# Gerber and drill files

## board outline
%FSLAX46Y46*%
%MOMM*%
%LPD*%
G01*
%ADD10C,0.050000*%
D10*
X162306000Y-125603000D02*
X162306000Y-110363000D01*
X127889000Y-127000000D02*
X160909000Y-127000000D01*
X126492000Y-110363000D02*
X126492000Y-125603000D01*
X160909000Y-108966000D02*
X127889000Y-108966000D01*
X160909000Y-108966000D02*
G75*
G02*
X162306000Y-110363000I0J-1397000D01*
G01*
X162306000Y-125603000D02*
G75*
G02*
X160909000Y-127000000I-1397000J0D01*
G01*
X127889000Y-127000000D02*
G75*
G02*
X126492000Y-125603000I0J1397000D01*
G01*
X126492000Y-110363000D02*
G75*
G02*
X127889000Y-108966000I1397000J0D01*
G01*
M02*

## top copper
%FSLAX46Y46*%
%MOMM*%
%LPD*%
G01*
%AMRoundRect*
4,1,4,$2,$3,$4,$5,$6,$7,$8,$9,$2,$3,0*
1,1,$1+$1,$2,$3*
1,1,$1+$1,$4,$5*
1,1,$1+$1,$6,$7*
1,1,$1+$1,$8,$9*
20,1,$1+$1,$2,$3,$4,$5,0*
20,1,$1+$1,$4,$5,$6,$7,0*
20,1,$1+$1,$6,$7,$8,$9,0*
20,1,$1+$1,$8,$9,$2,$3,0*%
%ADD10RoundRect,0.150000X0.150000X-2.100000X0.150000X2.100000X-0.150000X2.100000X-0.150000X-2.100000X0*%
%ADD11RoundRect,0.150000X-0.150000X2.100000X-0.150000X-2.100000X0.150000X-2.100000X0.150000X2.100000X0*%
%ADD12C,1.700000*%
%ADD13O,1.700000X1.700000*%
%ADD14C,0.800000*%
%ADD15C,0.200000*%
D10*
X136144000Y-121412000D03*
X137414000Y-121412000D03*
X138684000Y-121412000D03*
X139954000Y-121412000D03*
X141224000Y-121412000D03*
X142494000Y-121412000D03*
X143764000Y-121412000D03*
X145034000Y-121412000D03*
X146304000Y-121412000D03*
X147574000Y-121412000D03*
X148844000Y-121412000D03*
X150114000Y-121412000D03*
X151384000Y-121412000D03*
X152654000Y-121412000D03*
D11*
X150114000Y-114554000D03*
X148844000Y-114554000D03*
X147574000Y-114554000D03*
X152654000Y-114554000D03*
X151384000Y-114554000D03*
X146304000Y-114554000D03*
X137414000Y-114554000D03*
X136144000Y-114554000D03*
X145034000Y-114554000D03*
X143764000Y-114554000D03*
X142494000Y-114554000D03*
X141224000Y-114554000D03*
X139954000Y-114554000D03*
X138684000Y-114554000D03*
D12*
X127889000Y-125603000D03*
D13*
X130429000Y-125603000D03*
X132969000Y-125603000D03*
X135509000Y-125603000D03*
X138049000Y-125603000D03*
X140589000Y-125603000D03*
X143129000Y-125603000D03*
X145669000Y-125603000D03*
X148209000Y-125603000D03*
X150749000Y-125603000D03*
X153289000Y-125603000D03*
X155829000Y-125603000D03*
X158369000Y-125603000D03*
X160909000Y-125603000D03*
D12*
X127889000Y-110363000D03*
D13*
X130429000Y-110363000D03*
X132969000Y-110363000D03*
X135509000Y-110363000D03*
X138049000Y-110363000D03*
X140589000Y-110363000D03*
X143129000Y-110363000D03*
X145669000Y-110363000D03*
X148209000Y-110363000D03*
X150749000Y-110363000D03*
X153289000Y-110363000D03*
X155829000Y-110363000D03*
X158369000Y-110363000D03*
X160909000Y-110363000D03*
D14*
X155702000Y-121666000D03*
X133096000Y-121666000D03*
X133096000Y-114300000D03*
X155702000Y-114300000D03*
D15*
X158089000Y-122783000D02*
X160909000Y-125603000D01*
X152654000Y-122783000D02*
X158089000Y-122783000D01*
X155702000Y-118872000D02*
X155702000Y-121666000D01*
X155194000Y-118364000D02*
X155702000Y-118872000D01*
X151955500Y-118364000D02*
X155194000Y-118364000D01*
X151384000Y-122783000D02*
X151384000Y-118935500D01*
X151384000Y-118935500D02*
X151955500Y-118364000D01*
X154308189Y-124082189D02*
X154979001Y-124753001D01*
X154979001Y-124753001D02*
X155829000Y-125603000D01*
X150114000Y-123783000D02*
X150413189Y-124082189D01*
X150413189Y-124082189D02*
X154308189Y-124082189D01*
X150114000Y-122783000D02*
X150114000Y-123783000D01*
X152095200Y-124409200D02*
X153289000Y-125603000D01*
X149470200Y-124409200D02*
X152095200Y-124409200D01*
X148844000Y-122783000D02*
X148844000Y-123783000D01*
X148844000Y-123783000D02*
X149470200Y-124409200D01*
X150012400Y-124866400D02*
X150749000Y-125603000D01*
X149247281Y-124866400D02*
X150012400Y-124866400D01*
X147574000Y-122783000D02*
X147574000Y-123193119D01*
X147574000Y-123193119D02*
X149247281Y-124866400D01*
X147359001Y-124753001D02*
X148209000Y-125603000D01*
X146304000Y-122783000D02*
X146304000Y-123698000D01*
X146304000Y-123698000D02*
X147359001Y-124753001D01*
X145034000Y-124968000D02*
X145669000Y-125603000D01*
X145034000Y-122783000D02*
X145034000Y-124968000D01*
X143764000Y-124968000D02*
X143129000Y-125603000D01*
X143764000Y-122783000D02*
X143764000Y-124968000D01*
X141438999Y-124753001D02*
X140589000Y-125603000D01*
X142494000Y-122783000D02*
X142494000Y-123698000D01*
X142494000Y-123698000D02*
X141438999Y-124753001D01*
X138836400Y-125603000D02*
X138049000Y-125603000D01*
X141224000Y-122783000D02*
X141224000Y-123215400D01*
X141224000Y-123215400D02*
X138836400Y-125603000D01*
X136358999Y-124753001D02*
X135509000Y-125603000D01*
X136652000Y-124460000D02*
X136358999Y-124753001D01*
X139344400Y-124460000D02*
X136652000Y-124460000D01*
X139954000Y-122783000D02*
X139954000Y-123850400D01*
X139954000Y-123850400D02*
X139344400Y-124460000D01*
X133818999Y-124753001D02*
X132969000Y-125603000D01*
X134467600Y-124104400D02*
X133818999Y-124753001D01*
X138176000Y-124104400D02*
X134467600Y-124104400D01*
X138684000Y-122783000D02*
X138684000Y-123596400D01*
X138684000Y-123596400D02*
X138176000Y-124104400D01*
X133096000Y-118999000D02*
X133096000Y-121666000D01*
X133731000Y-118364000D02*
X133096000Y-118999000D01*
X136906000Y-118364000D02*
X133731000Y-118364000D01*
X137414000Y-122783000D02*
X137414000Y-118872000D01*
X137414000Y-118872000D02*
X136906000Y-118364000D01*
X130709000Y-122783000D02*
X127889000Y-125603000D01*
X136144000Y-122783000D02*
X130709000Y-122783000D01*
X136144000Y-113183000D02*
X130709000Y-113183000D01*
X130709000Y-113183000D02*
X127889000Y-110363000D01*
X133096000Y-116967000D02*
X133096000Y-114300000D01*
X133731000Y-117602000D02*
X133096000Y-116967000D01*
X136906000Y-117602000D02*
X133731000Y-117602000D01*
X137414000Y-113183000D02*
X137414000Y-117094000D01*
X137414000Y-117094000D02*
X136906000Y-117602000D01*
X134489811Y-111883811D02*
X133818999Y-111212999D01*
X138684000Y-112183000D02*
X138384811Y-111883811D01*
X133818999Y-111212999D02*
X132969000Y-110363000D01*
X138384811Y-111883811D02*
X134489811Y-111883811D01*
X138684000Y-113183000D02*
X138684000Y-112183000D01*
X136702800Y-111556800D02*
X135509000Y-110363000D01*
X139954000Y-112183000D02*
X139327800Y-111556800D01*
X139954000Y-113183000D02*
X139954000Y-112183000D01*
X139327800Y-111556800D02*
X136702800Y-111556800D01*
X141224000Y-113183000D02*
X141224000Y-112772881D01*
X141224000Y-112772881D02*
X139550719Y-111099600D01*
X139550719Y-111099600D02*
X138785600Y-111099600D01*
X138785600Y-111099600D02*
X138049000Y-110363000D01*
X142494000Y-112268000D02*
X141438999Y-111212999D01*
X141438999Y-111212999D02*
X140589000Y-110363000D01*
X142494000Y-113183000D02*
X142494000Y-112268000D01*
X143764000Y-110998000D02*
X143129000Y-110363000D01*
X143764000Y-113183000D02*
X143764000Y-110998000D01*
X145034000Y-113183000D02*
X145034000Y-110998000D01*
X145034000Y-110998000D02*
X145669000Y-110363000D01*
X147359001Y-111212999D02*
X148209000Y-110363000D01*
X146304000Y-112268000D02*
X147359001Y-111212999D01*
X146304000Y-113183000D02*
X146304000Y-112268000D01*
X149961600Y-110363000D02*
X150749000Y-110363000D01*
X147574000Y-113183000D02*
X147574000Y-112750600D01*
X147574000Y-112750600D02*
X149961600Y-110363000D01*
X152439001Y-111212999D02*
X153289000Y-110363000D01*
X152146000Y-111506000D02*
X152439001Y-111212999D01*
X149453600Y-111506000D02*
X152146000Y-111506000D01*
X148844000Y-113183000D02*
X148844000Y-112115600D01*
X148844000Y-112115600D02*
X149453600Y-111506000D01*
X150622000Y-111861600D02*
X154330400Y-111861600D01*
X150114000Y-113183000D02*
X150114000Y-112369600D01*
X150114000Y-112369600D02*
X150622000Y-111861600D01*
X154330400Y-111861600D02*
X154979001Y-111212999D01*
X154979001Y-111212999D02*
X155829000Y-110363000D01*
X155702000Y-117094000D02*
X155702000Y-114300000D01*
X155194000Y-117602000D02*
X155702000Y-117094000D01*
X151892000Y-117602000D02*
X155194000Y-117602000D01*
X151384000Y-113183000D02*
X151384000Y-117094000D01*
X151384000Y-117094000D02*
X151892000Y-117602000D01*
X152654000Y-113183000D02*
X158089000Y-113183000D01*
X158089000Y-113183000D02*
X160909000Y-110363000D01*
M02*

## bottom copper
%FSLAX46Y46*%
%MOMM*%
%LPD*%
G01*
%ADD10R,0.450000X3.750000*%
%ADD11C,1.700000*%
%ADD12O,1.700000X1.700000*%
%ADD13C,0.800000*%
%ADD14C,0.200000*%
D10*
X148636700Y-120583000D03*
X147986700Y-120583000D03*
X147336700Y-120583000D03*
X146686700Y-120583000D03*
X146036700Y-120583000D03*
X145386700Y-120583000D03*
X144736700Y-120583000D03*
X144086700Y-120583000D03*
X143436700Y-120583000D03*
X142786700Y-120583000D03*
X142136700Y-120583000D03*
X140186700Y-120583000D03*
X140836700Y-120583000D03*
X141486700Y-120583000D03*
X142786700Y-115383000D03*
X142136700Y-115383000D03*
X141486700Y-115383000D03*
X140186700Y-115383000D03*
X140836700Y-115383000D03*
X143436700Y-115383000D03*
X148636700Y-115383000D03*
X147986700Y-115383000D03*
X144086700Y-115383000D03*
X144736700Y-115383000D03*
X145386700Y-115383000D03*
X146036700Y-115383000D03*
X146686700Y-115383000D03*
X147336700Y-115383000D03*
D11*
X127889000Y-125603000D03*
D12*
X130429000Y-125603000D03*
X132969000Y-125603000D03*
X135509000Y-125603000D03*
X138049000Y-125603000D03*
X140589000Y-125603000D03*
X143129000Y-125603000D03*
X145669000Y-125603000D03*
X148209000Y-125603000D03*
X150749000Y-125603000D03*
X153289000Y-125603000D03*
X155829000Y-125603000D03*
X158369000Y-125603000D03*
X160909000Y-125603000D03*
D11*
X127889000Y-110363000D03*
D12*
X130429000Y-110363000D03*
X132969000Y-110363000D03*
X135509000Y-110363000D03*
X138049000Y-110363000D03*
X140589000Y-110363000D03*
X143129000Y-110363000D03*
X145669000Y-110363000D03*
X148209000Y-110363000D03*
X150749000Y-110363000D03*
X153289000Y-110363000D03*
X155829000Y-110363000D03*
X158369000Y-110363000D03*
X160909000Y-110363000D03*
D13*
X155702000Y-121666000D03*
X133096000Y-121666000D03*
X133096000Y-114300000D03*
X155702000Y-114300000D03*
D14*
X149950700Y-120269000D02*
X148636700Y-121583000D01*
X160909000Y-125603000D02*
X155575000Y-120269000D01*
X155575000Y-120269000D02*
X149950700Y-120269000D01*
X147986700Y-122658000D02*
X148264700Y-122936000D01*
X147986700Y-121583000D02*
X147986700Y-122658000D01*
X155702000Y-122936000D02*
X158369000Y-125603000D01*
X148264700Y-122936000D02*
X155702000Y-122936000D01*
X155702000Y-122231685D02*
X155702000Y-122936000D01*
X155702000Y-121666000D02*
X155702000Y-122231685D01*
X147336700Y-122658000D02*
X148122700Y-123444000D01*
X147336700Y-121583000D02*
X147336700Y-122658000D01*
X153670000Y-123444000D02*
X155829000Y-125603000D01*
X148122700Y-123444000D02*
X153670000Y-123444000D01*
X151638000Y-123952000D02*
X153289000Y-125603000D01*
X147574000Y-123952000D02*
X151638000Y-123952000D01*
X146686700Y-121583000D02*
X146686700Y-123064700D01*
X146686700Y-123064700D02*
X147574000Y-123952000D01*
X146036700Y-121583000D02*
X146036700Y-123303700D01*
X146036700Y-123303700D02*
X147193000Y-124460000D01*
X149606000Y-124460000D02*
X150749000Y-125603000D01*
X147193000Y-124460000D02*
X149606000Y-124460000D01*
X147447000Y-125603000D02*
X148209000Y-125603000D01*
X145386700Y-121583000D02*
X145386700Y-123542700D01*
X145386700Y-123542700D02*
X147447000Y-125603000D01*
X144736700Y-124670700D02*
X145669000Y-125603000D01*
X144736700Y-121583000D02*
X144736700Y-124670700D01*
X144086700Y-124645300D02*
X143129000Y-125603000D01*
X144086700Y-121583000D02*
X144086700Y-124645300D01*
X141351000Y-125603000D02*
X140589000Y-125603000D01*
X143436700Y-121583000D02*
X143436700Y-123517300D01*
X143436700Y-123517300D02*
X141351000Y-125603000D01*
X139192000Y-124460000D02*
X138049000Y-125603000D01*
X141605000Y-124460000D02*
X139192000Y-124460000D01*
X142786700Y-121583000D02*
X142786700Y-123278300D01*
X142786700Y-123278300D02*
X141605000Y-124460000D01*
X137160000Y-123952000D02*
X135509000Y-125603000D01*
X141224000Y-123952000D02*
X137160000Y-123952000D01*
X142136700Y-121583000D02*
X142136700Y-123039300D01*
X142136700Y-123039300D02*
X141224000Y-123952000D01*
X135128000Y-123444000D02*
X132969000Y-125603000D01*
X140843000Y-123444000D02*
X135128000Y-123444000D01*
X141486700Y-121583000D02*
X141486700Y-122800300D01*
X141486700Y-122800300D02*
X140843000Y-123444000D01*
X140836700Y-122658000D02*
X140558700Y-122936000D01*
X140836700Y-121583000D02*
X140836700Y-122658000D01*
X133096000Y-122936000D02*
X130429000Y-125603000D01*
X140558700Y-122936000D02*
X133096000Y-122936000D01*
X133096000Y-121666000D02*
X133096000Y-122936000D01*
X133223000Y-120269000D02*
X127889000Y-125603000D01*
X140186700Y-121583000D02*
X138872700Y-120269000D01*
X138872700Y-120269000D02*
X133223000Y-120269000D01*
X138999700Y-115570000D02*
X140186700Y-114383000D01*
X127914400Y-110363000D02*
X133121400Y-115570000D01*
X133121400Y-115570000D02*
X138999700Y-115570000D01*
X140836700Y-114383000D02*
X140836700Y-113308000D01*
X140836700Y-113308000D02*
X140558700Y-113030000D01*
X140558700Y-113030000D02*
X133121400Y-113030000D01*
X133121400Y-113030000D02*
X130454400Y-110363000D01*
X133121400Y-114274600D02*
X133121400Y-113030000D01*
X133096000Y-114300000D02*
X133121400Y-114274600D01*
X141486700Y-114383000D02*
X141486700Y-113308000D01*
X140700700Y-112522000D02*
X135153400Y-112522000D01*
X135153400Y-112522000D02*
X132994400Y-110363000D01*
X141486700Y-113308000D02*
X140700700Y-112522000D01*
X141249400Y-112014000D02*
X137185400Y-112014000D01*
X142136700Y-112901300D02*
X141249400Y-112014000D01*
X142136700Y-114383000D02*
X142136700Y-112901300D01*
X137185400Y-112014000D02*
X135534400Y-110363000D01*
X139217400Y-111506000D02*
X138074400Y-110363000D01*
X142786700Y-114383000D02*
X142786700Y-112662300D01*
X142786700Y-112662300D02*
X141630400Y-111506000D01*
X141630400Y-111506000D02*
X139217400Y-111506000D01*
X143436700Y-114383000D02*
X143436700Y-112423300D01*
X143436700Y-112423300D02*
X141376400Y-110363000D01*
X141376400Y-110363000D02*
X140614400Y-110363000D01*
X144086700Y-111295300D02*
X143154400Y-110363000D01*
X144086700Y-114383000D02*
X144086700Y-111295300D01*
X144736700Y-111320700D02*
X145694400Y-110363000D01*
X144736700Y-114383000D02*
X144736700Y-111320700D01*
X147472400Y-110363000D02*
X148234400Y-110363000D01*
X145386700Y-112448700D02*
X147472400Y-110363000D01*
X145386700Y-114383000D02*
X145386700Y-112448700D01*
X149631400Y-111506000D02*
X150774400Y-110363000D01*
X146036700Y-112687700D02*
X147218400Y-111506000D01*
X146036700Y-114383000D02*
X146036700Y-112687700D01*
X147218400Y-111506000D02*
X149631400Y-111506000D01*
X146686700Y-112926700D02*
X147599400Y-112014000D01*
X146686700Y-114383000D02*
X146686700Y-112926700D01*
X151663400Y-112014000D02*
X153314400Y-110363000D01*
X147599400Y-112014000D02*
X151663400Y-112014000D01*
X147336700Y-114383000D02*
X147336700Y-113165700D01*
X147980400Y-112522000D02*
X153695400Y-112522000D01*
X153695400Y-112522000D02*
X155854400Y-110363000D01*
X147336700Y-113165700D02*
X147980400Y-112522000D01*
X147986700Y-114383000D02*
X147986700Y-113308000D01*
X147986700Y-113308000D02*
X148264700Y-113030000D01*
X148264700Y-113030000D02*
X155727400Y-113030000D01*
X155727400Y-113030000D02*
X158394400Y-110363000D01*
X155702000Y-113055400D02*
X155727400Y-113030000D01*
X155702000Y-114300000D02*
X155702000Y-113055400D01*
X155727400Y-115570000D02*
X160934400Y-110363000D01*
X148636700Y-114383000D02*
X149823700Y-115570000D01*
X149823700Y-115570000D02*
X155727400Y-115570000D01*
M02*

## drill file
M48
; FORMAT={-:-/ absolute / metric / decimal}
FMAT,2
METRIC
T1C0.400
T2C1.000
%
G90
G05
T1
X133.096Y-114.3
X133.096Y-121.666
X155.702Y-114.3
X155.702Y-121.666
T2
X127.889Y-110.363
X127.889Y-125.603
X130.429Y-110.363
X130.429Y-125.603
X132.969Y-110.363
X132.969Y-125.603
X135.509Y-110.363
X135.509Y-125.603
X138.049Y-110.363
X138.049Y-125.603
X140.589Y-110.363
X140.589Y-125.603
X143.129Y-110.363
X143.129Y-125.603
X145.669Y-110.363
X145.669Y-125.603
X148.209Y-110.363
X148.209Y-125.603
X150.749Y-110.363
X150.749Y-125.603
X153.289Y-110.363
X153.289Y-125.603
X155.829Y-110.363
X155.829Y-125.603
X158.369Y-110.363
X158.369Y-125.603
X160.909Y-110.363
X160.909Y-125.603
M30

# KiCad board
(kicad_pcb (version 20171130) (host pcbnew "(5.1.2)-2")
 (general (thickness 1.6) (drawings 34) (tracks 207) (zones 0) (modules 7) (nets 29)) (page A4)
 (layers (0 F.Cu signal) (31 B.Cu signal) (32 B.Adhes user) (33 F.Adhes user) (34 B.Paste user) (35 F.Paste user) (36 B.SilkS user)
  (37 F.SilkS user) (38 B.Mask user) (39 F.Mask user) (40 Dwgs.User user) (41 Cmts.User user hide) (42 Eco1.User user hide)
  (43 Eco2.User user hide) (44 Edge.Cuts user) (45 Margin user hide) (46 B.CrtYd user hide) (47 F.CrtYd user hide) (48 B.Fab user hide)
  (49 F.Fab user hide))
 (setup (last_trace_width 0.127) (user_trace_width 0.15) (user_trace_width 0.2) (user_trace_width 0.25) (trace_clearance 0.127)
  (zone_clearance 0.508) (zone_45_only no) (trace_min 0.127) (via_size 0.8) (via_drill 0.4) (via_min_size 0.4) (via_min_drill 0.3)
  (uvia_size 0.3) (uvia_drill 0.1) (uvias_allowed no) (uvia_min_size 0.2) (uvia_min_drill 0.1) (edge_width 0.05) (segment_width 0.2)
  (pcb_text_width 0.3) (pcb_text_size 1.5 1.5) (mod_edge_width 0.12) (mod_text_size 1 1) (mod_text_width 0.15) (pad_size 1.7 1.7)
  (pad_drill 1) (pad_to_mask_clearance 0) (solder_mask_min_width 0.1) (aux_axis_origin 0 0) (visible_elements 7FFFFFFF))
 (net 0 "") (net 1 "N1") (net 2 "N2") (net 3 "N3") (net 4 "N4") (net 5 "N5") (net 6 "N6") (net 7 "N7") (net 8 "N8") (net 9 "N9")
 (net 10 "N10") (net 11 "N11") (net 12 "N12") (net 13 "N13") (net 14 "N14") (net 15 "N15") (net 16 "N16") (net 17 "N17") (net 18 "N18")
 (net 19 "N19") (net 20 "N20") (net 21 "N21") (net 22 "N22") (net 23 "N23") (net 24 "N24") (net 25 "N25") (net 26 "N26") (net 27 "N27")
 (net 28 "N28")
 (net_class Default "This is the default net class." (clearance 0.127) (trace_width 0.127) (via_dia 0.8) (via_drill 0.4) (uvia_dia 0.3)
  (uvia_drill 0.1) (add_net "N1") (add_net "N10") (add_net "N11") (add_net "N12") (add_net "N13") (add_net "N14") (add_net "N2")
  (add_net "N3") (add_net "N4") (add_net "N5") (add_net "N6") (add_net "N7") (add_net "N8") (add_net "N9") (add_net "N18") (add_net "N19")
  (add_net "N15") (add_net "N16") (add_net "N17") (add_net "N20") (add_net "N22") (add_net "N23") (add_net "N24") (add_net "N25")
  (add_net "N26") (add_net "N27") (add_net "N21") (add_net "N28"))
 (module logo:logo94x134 (layer B.Cu) (at 157.226 117.983 180)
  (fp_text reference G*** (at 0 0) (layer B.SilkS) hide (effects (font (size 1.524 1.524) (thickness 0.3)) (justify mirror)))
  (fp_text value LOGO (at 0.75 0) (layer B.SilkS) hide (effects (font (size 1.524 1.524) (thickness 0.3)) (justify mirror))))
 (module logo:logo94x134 (layer F.Cu) (at 130.429 117.983)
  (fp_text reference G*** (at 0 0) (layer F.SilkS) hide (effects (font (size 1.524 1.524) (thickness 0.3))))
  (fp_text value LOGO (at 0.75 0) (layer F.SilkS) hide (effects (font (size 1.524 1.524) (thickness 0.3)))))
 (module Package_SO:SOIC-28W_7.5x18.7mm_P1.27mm (layer F.Cu) (at 144.399 117.983 90)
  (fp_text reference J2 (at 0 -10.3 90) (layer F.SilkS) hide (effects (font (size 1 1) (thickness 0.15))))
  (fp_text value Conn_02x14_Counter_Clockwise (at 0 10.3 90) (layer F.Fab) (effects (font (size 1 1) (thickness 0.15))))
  (pad 1 smd roundrect (at -3.429 -8.255 90) (size 4.5 0.6) (layers F.Cu F.Paste F.Mask) (roundrect_rratio 0.25) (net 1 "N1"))
  (pad 2 smd roundrect (at -3.429 -6.985 90) (size 4.5 0.6) (layers F.Cu F.Paste F.Mask) (roundrect_rratio 0.25) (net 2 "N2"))
  (pad 3 smd roundrect (at -3.429 -5.715 90) (size 4.5 0.6) (layers F.Cu F.Paste F.Mask) (roundrect_rratio 0.25) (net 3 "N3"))
  (pad 4 smd roundrect (at -3.429 -4.445 90) (size 4.5 0.6) (layers F.Cu F.Paste F.Mask) (roundrect_rratio 0.25) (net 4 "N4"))
  (pad 5 smd roundrect (at -3.429 -3.175 90) (size 4.5 0.6) (layers F.Cu F.Paste F.Mask) (roundrect_rratio 0.25) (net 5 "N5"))
  (pad 6 smd roundrect (at -3.429 -1.905 90) (size 4.5 0.6) (layers F.Cu F.Paste F.Mask) (roundrect_rratio 0.25) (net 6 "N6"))
  (pad 7 smd roundrect (at -3.429 -0.635 90) (size 4.5 0.6) (layers F.Cu F.Paste F.Mask) (roundrect_rratio 0.25) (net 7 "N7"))
  (pad 8 smd roundrect (at -3.429 0.635 90) (size 4.5 0.6) (layers F.Cu F.Paste F.Mask) (roundrect_rratio 0.25) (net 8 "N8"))
  (pad 9 smd roundrect (at -3.429 1.905 90) (size 4.5 0.6) (layers F.Cu F.Paste F.Mask) (roundrect_rratio 0.25) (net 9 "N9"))
  (pad 10 smd roundrect (at -3.429 3.175 90) (size 4.5 0.6) (layers F.Cu F.Paste F.Mask) (roundrect_rratio 0.25) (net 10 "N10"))
  (pad 11 smd roundrect (at -3.429 4.445 90) (size 4.5 0.6) (layers F.Cu F.Paste F.Mask) (roundrect_rratio 0.25) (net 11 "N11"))
  (pad 12 smd roundrect (at -3.429 5.715 90) (size 4.5 0.6) (layers F.Cu F.Paste F.Mask) (roundrect_rratio 0.25) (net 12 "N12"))
  (pad 13 smd roundrect (at -3.429 6.985 90) (size 4.5 0.6) (layers F.Cu F.Paste F.Mask) (roundrect_rratio 0.25) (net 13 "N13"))
  (pad 14 smd roundrect (at -3.429 8.255 90) (size 4.5 0.6) (layers F.Cu F.Paste F.Mask) (roundrect_rratio 0.25) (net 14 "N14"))
  (pad 17 smd roundrect (at 3.429 5.715 270) (size 4.5 0.6) (layers F.Cu F.Paste F.Mask) (roundrect_rratio 0.25) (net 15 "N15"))
  (pad 18 smd roundrect (at 3.429 4.445 270) (size 4.5 0.6) (layers F.Cu F.Paste F.Mask) (roundrect_rratio 0.25) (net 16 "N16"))
  (pad 19 smd roundrect (at 3.429 3.175 270) (size 4.5 0.6) (layers F.Cu F.Paste F.Mask) (roundrect_rratio 0.25) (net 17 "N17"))
  (pad 15 smd roundrect (at 3.429 8.255 270) (size 4.5 0.6) (layers F.Cu F.Paste F.Mask) (roundrect_rratio 0.25) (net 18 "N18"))
  (pad 16 smd roundrect (at 3.429 6.985 270) (size 4.5 0.6) (layers F.Cu F.Paste F.Mask) (roundrect_rratio 0.25) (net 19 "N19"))
  (pad 20 smd roundrect (at 3.429 1.905 270) (size 4.5 0.6) (layers F.Cu F.Paste F.Mask) (roundrect_rratio 0.25) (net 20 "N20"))
  (pad 27 smd roundrect (at 3.429 -6.985 270) (size 4.5 0.6) (layers F.Cu F.Paste F.Mask) (roundrect_rratio 0.25) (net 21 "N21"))
  (pad 8 smd roundrect (at 3.429 -8.255 270) (size 4.5 0.6) (layers F.Cu F.Paste F.Mask) (roundrect_rratio 0.25) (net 8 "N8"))
  (pad 21 smd roundrect (at 3.429 0.635 270) (size 4.5 0.6) (layers F.Cu F.Paste F.Mask) (roundrect_rratio 0.25) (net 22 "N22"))
  (pad 22 smd roundrect (at 3.429 -0.635 270) (size 4.5 0.6) (layers F.Cu F.Paste F.Mask) (roundrect_rratio 0.25) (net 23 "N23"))
  (pad 23 smd roundrect (at 3.429 -1.905 270) (size 4.5 0.6) (layers F.Cu F.Paste F.Mask) (roundrect_rratio 0.25) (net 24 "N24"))
  (pad 24 smd roundrect (at 3.429 -3.175 270) (size 4.5 0.6) (layers F.Cu F.Paste F.Mask) (roundrect_rratio 0.25) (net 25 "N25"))
  (pad 25 smd roundrect (at 3.429 -4.445 270) (size 4.5 0.6) (layers F.Cu F.Paste F.Mask) (roundrect_rratio 0.25) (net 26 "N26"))
  (pad 26 smd roundrect (at 3.429 -5.715 270) (size 4.5 0.6) (layers F.Cu F.Paste F.Mask) (roundrect_rratio 0.25) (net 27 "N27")))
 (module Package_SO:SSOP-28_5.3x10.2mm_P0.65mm (layer B.Cu) (at 144.4117 117.983 90)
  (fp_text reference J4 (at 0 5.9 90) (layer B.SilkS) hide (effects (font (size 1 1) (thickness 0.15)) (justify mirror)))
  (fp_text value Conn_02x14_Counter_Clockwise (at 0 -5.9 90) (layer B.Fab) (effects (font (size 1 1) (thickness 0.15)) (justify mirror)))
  (pad 1 smd rect (at -2.6 4.225 90) (size 3.75 0.45) (layers B.Cu B.Paste B.Mask) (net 14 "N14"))
  (pad 2 smd rect (at -2.6 3.575 90) (size 3.75 0.45) (layers B.Cu B.Paste B.Mask) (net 13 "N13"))
  (pad 3 smd rect (at -2.6 2.925 90) (size 3.75 0.45) (layers B.Cu B.Paste B.Mask) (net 12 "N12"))
  (pad 4 smd rect (at -2.6 2.275 90) (size 3.75 0.45) (layers B.Cu B.Paste B.Mask) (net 11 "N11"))
  (pad 5 smd rect (at -2.6 1.625 90) (size 3.75 0.45) (layers B.Cu B.Paste B.Mask) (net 10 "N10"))
  (pad 6 smd rect (at -2.6 0.975 90) (size 3.75 0.45) (layers B.Cu B.Paste B.Mask) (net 9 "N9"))
  (pad 7 smd rect (at -2.6 0.325 90) (size 3.75 0.45) (layers B.Cu B.Paste B.Mask) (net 8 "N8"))
  (pad 8 smd rect (at -2.6 -0.325 90) (size 3.75 0.45) (layers B.Cu B.Paste B.Mask) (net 7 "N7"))
  (pad 9 smd rect (at -2.6 -0.975 90) (size 3.75 0.45) (layers B.Cu B.Paste B.Mask) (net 6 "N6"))
  (pad 10 smd rect (at -2.6 -1.625 90) (size 3.75 0.45) (layers B.Cu B.Paste B.Mask) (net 5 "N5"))
  (pad 11 smd rect (at -2.6 -2.275 90) (size 3.75 0.45) (layers B.Cu B.Paste B.Mask) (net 4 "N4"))
  (pad 14 smd rect (at -2.6 -4.225 90) (size 3.75 0.45) (layers B.Cu B.Paste B.Mask) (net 1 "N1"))
  (pad 13 smd rect (at -2.6 -3.575 90) (size 3.75 0.45) (layers B.Cu B.Paste B.Mask) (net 2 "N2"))
  (pad 12 smd rect (at -2.6 -2.925 90) (size 3.75 0.45) (layers B.Cu B.Paste B.Mask) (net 3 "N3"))
  (pad 19 smd rect (at 2.6 -1.625 270) (size 3.75 0.45) (layers B.Cu B.Paste B.Mask) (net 25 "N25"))
  (pad 18 smd rect (at 2.6 -2.275 270) (size 3.75 0.45) (layers B.Cu B.Paste B.Mask) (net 26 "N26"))
  (pad 17 smd rect (at 2.6 -2.925 270) (size 3.75 0.45) (layers B.Cu B.Paste B.Mask) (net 27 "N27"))
  (pad 15 smd rect (at 2.6 -4.225 270) (size 3.75 0.45) (layers B.Cu B.Paste B.Mask) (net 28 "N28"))
  (pad 16 smd rect (at 2.6 -3.575 270) (size 3.75 0.45) (layers B.Cu B.Paste B.Mask) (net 21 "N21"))
  (pad 20 smd rect (at 2.6 -0.975 270) (size 3.75 0.45) (layers B.Cu B.Paste B.Mask) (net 24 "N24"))
  (pad 28 smd rect (at 2.6 4.225 270) (size 3.75 0.45) (layers B.Cu B.Paste B.Mask) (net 18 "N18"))
  (pad 27 smd rect (at 2.6 3.575 270) (size 3.75 0.45) (layers B.Cu B.Paste B.Mask) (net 19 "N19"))
  (pad 21 smd rect (at 2.6 -0.325 270) (size 3.75 0.45) (layers B.Cu B.Paste B.Mask) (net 23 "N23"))
  (pad 22 smd rect (at 2.6 0.325 270) (size 3.75 0.45) (layers B.Cu B.Paste B.Mask) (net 22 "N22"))
  (pad 23 smd rect (at 2.6 0.975 270) (size 3.75 0.45) (layers B.Cu B.Paste B.Mask) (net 20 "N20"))
  (pad 24 smd rect (at 2.6 1.625 270) (size 3.75 0.45) (layers B.Cu B.Paste B.Mask) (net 17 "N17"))
  (pad 25 smd rect (at 2.6 2.275 270) (size 3.75 0.45) (layers B.Cu B.Paste B.Mask) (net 16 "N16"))
  (pad 26 smd rect (at 2.6 2.925 270) (size 3.75 0.45) (layers B.Cu B.Paste B.Mask) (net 15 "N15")))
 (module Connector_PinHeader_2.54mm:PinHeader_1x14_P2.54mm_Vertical (layer B.Cu) (at 127.889 125.603 270)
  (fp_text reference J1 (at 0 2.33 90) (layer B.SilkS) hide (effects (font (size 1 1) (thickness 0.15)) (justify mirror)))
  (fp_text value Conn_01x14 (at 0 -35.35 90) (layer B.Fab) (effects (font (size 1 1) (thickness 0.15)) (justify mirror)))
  (pad 1 thru_hole circle (at 0 0 270) (size 1.7 1.7) (drill 1) (layers *.Cu *.Mask) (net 1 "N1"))
  (pad 2 thru_hole oval (at 0 -2.54 270) (size 1.7 1.7) (drill 1) (layers *.Cu *.Mask) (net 2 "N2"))
  (pad 3 thru_hole oval (at 0 -5.08 270) (size 1.7 1.7) (drill 1) (layers *.Cu *.Mask) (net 3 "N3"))
  (pad 4 thru_hole oval (at 0 -7.62 270) (size 1.7 1.7) (drill 1) (layers *.Cu *.Mask) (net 4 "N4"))
  (pad 5 thru_hole oval (at 0 -10.16 270) (size 1.7 1.7) (drill 1) (layers *.Cu *.Mask) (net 5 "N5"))
  (pad 6 thru_hole oval (at 0 -12.7 270) (size 1.7 1.7) (drill 1) (layers *.Cu *.Mask) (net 6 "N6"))
  (pad 7 thru_hole oval (at 0 -15.24 270) (size 1.7 1.7) (drill 1) (layers *.Cu *.Mask) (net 7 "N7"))
  (pad 8 thru_hole oval (at 0 -17.78 270) (size 1.7 1.7) (drill 1) (layers *.Cu *.Mask) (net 8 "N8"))
  (pad 9 thru_hole oval (at 0 -20.32 270) (size 1.7 1.7) (drill 1) (layers *.Cu *.Mask) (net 9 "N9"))
  (pad 10 thru_hole oval (at 0 -22.86 270) (size 1.7 1.7) (drill 1) (layers *.Cu *.Mask) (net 10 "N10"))
  (pad 11 thru_hole oval (at 0 -25.4 270) (size 1.7 1.7) (drill 1) (layers *.Cu *.Mask) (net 11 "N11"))
  (pad 12 thru_hole oval (at 0 -27.94 270) (size 1.7 1.7) (drill 1) (layers *.Cu *.Mask) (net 12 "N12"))
  (pad 13 thru_hole oval (at 0 -30.48 270) (size 1.7 1.7) (drill 1) (layers *.Cu *.Mask) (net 13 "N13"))
  (pad 14 thru_hole oval (at 0 -33.02 270) (size 1.7 1.7) (drill 1) (layers *.Cu *.Mask) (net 14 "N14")))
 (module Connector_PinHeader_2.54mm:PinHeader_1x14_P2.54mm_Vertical (layer B.Cu) (at 127.889 110.363 270)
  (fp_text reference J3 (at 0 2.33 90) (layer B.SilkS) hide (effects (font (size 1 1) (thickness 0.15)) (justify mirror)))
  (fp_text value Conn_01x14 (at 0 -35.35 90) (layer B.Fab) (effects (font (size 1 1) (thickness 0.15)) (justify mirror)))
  (pad 1 thru_hole circle (at 0 0 270) (size 1.7 1.7) (drill 1) (layers *.Cu *.Mask) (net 28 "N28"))
  (pad 2 thru_hole oval (at 0 -2.54 270) (size 1.7 1.7) (drill 1) (layers *.Cu *.Mask) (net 21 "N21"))
  (pad 3 thru_hole oval (at 0 -5.08 270) (size 1.7 1.7) (drill 1) (layers *.Cu *.Mask) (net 27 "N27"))
  (pad 4 thru_hole oval (at 0 -7.62 270) (size 1.7 1.7) (drill 1) (layers *.Cu *.Mask) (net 26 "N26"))
  (pad 5 thru_hole oval (at 0 -10.16 270) (size 1.7 1.7) (drill 1) (layers *.Cu *.Mask) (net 25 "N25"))
  (pad 6 thru_hole oval (at 0 -12.7 270) (size 1.7 1.7) (drill 1) (layers *.Cu *.Mask) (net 24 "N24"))
  (pad 7 thru_hole oval (at 0 -15.24 270) (size 1.7 1.7) (drill 1) (layers *.Cu *.Mask) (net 23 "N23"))
  (pad 8 thru_hole oval (at 0 -17.78 270) (size 1.7 1.7) (drill 1) (layers *.Cu *.Mask) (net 22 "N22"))
  (pad 9 thru_hole oval (at 0 -20.32 270) (size 1.7 1.7) (drill 1) (layers *.Cu *.Mask) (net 20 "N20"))
  (pad 10 thru_hole oval (at 0 -22.86 270) (size 1.7 1.7) (drill 1) (layers *.Cu *.Mask) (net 17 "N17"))
  (pad 11 thru_hole oval (at 0 -25.4 270) (size 1.7 1.7) (drill 1) (layers *.Cu *.Mask) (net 16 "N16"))
  (pad 12 thru_hole oval (at 0 -27.94 270) (size 1.7 1.7) (drill 1) (layers *.Cu *.Mask) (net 15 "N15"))
  (pad 13 thru_hole oval (at 0 -30.48 270) (size 1.7 1.7) (drill 1) (layers *.Cu *.Mask) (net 19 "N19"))
  (pad 14 thru_hole oval (at 0 -33.02 270) (size 1.7 1.7) (drill 1) (layers *.Cu *.Mask) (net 18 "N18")))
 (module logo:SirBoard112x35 (layer B.Cu) (at 136.144 117.983 90)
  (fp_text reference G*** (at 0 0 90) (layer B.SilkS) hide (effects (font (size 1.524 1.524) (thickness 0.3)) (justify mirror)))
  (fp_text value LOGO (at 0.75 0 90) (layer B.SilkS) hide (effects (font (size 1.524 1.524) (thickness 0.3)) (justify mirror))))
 (gr_line (start 162.306 125.603) (end 162.306 110.363) (layer Edge.Cuts) (width 0.05))
 (gr_line (start 127.889 127) (end 160.909 127) (layer Edge.Cuts) (width 0.05))
 (gr_line (start 126.492 110.363) (end 126.492 125.603) (layer Edge.Cuts) (width 0.05))
 (gr_line (start 160.909 108.966) (end 127.889 108.966) (layer Edge.Cuts) (width 0.05))
 (gr_arc (start 160.909 110.363) (end 162.306 110.363) (angle -90) (layer Edge.Cuts) (width 0.05))
 (gr_arc (start 160.909 125.603) (end 160.909 127) (angle -90) (layer Edge.Cuts) (width 0.05))
 (gr_arc (start 127.889 125.603) (end 126.492 125.603) (angle -90) (layer Edge.Cuts) (width 0.05))
 (gr_arc (start 127.889 110.363) (end 127.889 108.966) (angle -90) (layer Edge.Cuts) (width 0.05))
 (segment (start 158.089 122.783) (end 160.909 125.603) (width 0.2) (layer F.Cu) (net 14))
 (segment (start 152.654 122.783) (end 158.089 122.783) (width 0.2) (layer F.Cu) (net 14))
 (segment (start 149.9507 120.269) (end 148.6367 121.583) (width 0.2) (layer B.Cu) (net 14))
 (segment (start 160.909 125.603) (end 155.575 120.269) (width 0.2) (layer B.Cu) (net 14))
 (segment (start 155.575 120.269) (end 149.9507 120.269) (width 0.2) (layer B.Cu) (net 14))
 (segment (start 147.9867 122.658) (end 148.2647 122.936) (width 0.2) (layer B.Cu) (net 13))
 (segment (start 147.9867 121.583) (end 147.9867 122.658) (width 0.2) (layer B.Cu) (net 13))
 (segment (start 155.702 122.936) (end 158.369 125.603) (width 0.2) (layer B.Cu) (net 13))
 (segment (start 148.2647 122.936) (end 155.702 122.936) (width 0.2) (layer B.Cu) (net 13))
 (via (at 155.702 121.666) (size 0.8) (drill 0.4) (layers F.Cu B.Cu) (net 13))
 (segment (start 155.702 122.231685) (end 155.702 122.936) (width 0.2) (layer B.Cu) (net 13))
 (segment (start 155.702 121.666) (end 155.702 122.231685) (width 0.2) (layer B.Cu) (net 13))
 (segment (start 155.702 118.872) (end 155.702 121.666) (width 0.2) (layer F.Cu) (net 13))
 (segment (start 155.194 118.364) (end 155.702 118.872) (width 0.2) (layer F.Cu) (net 13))
 (segment (start 151.9555 118.364) (end 155.194 118.364) (width 0.2) (layer F.Cu) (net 13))
 (segment (start 151.384 122.783) (end 151.384 118.9355) (width 0.2) (layer F.Cu) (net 13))
 (segment (start 151.384 118.9355) (end 151.9555 118.364) (width 0.2) (layer F.Cu) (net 13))
 (segment (start 147.3367 122.658) (end 148.1227 123.444) (width 0.2) (layer B.Cu) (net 12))
 (segment (start 147.3367 121.583) (end 147.3367 122.658) (width 0.2) (layer B.Cu) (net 12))
 (segment (start 153.67 123.444) (end 155.829 125.603) (width 0.2) (layer B.Cu) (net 12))
 (segment (start 148.1227 123.444) (end 153.67 123.444) (width 0.2) (layer B.Cu) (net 12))
 (segment (start 154.308189 124.082189) (end 154.979001 124.753001) (width 0.2) (layer F.Cu) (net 12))
 (segment (start 154.979001 124.753001) (end 155.829 125.603) (width 0.2) (layer F.Cu) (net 12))
 (segment (start 150.114 123.783) (end 150.413189 124.082189) (width 0.2) (layer F.Cu) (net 12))
 (segment (start 150.413189 124.082189) (end 154.308189 124.082189) (width 0.2) (layer F.Cu) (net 12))
 (segment (start 150.114 122.783) (end 150.114 123.783) (width 0.2) (layer F.Cu) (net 12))
 (segment (start 151.638 123.952) (end 153.289 125.603) (width 0.2) (layer B.Cu) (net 11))
 (segment (start 147.574 123.952) (end 151.638 123.952) (width 0.2) (layer B.Cu) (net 11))
 (segment (start 146.6867 121.583) (end 146.6867 123.0647) (width 0.2) (layer B.Cu) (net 11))
 (segment (start 146.6867 123.0647) (end 147.574 123.952) (width 0.2) (layer B.Cu) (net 11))
 (segment (start 152.0952 124.4092) (end 153.289 125.603) (width 0.2) (layer F.Cu) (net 11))
 (segment (start 149.4702 124.4092) (end 152.0952 124.4092) (width 0.2) (layer F.Cu) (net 11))
 (segment (start 148.844 122.783) (end 148.844 123.783) (width 0.2) (layer F.Cu) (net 11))
 (segment (start 148.844 123.783) (end 149.4702 124.4092) (width 0.2) (layer F.Cu) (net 11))
 (segment (start 146.0367 121.583) (end 146.0367 123.3037) (width 0.2) (layer B.Cu) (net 10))
 (segment (start 146.0367 123.3037) (end 147.193 124.46) (width 0.2) (layer B.Cu) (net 10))
 (segment (start 149.606 124.46) (end 150.749 125.603) (width 0.2) (layer B.Cu) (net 10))
 (segment (start 147.193 124.46) (end 149.606 124.46) (width 0.2) (layer B.Cu) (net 10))
 (segment (start 150.0124 124.8664) (end 150.749 125.603) (width 0.2) (layer F.Cu) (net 10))
 (segment (start 149.247281 124.8664) (end 150.0124 124.8664) (width 0.2) (layer F.Cu) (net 10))
 (segment (start 147.574 122.783) (end 147.574 123.193119) (width 0.2) (layer F.Cu) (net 10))
 (segment (start 147.574 123.193119) (end 149.247281 124.8664) (width 0.2) (layer F.Cu) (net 10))
 (segment (start 147.447 125.603) (end 148.209 125.603) (width 0.2) (layer B.Cu) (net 9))
 (segment (start 145.3867 121.583) (end 145.3867 123.5427) (width 0.2) (layer B.Cu) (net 9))
 (segment (start 145.3867 123.5427) (end 147.447 125.603) (width 0.2) (layer B.Cu) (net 9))
 (segment (start 147.359001 124.753001) (end 148.209 125.603) (width 0.2) (layer F.Cu) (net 9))
 (segment (start 146.304 122.783) (end 146.304 123.698) (width 0.2) (layer F.Cu) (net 9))
 (segment (start 146.304 123.698) (end 147.359001 124.753001) (width 0.2) (layer F.Cu) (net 9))
 (segment (start 144.7367 124.6707) (end 145.669 125.603) (width 0.2) (layer B.Cu) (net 8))
 (segment (start 144.7367 121.583) (end 144.7367 124.6707) (width 0.2) (layer B.Cu) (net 8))
 (segment (start 145.034 124.968) (end 145.669 125.603) (width 0.2) (layer F.Cu) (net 8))
 (segment (start 145.034 122.783) (end 145.034 124.968) (width 0.2) (layer F.Cu) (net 8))
 (segment (start 144.0867 124.6453) (end 143.129 125.603) (width 0.2) (layer B.Cu) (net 7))
 (segment (start 144.0867 121.583) (end 144.0867 124.6453) (width 0.2) (layer B.Cu) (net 7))
 (segment (start 143.764 124.968) (end 143.129 125.603) (width 0.2) (layer F.Cu) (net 7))
 (segment (start 143.764 122.783) (end 143.764 124.968) (width 0.2) (layer F.Cu) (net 7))
 (segment (start 141.351 125.603) (end 140.589 125.603) (width 0.2) (layer B.Cu) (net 6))
 (segment (start 143.4367 121.583) (end 143.4367 123.5173) (width 0.2) (layer B.Cu) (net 6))
 (segment (start 143.4367 123.5173) (end 141.351 125.603) (width 0.2) (layer B.Cu) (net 6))
 (segment (start 141.438999 124.753001) (end 140.589 125.603) (width 0.2) (layer F.Cu) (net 6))
 (segment (start 142.494 122.783) (end 142.494 123.698) (width 0.2) (layer F.Cu) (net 6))
 (segment (start 142.494 123.698) (end 141.438999 124.753001) (width 0.2) (layer F.Cu) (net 6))
 (segment (start 139.192 124.46) (end 138.049 125.603) (width 0.2) (layer B.Cu) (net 5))
 (segment (start 141.605 124.46) (end 139.192 124.46) (width 0.2) (layer B.Cu) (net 5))
 (segment (start 142.7867 121.583) (end 142.7867 123.2783) (width 0.2) (layer B.Cu) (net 5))
 (segment (start 142.7867 123.2783) (end 141.605 124.46) (width 0.2) (layer B.Cu) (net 5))
 (segment (start 138.8364 125.603) (end 138.049 125.603) (width 0.2) (layer F.Cu) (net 5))
 (segment (start 141.224 122.783) (end 141.224 123.2154) (width 0.2) (layer F.Cu) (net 5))
 (segment (start 141.224 123.2154) (end 138.8364 125.603) (width 0.2) (layer F.Cu) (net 5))
 (segment (start 137.16 123.952) (end 135.509 125.603) (width 0.2) (layer B.Cu) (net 4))
 (segment (start 141.224 123.952) (end 137.16 123.952) (width 0.2) (layer B.Cu) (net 4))
 (segment (start 142.1367 121.583) (end 142.1367 123.0393) (width 0.2) (layer B.Cu) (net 4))
 (segment (start 142.1367 123.0393) (end 141.224 123.952) (width 0.2) (layer B.Cu) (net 4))
 (segment (start 136.358999 124.753001) (end 135.509 125.603) (width 0.2) (layer F.Cu) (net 4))
 (segment (start 136.652 124.46) (end 136.358999 124.753001) (width 0.2) (layer F.Cu) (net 4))
 (segment (start 139.3444 124.46) (end 136.652 124.46) (width 0.2) (layer F.Cu) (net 4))
 (segment (start 139.954 122.783) (end 139.954 123.8504) (width 0.2) (layer F.Cu) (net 4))
 (segment (start 139.954 123.8504) (end 139.3444 124.46) (width 0.2) (layer F.Cu) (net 4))
 (segment (start 135.128 123.444) (end 132.969 125.603) (width 0.2) (layer B.Cu) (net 3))
 (segment (start 140.843 123.444) (end 135.128 123.444) (width 0.2) (layer B.Cu) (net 3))
 (segment (start 141.4867 121.583) (end 141.4867 122.8003) (width 0.2) (layer B.Cu) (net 3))
 (segment (start 141.4867 122.8003) (end 140.843 123.444) (width 0.2) (layer B.Cu) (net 3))
 (segment (start 133.818999 124.753001) (end 132.969 125.603) (width 0.2) (layer F.Cu) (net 3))
 (segment (start 134.4676 124.1044) (end 133.818999 124.753001) (width 0.2) (layer F.Cu) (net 3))
 (segment (start 138.176 124.1044) (end 134.4676 124.1044) (width 0.2) (layer F.Cu) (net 3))
 (segment (start 138.684 122.783) (end 138.684 123.5964) (width 0.2) (layer F.Cu) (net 3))
 (segment (start 138.684 123.5964) (end 138.176 124.1044) (width 0.2) (layer F.Cu) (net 3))
 (segment (start 140.8367 122.658) (end 140.5587 122.936) (width 0.2) (layer B.Cu) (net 2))
 (segment (start 140.8367 121.583) (end 140.8367 122.658) (width 0.2) (layer B.Cu) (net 2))
 (segment (start 133.096 122.936) (end 130.429 125.603) (width 0.2) (layer B.Cu) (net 2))
 (segment (start 140.5587 122.936) (end 133.096 122.936) (width 0.2) (layer B.Cu) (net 2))
 (via (at 133.096 121.666) (size 0.8) (drill 0.4) (layers F.Cu B.Cu) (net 2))
 (segment (start 133.096 121.666) (end 133.096 122.936) (width 0.2) (layer B.Cu) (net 2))
 (segment (start 133.096 118.999) (end 133.096 121.666) (width 0.2) (layer F.Cu) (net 2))
 (segment (start 133.731 118.364) (end 133.096 118.999) (width 0.2) (layer F.Cu) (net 2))
 (segment (start 136.906 118.364) (end 133.731 118.364) (width 0.2) (layer F.Cu) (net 2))
 (segment (start 137.414 122.783) (end 137.414 118.872) (width 0.2) (layer F.Cu) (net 2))
 (segment (start 137.414 118.872) (end 136.906 118.364) (width 0.2) (layer F.Cu) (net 2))
 (segment (start 130.709 122.783) (end 127.889 125.603) (width 0.2) (layer F.Cu) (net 1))
 (segment (start 136.144 122.783) (end 130.709 122.783) (width 0.2) (layer F.Cu) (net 1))
 (segment (start 133.223 120.269) (end 127.889 125.603) (width 0.2) (layer B.Cu) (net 1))
 (segment (start 140.1867 121.583) (end 138.8727 120.269) (width 0.2) (layer B.Cu) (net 1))
 (segment (start 138.8727 120.269) (end 133.223 120.269) (width 0.2) (layer B.Cu) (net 1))
 (segment (start 136.144 113.183) (end 130.709 113.183) (width 0.2) (layer F.Cu) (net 28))
 (segment (start 130.709 113.183) (end 127.889 110.363) (width 0.2) (layer F.Cu) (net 28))
 (segment (start 138.9997 115.57) (end 140.1867 114.383) (width 0.2) (layer B.Cu) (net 28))
 (segment (start 127.9144 110.363) (end 133.1214 115.57) (width 0.2) (layer B.Cu) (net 28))
 (segment (start 133.1214 115.57) (end 138.9997 115.57) (width 0.2) (layer B.Cu) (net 28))
 (via (at 133.096 114.3) (size 0.8) (drill 0.4) (layers F.Cu B.Cu) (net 21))
 (segment (start 140.8367 114.383) (end 140.8367 113.308) (width 0.2) (layer B.Cu) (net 21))
 (segment (start 140.8367 113.308) (end 140.5587 113.03) (width 0.2) (layer B.Cu) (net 21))
 (segment (start 140.5587 113.03) (end 133.1214 113.03) (width 0.2) (layer B.Cu) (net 21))
 (segment (start 133.1214 113.03) (end 130.4544 110.363) (width 0.2) (layer B.Cu) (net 21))
 (segment (start 133.1214 114.2746) (end 133.1214 113.03) (width 0.2) (layer B.Cu) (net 21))
 (segment (start 133.096 114.3) (end 133.1214 114.2746) (width 0.2) (layer B.Cu) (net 21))
 (segment (start 133.096 116.967) (end 133.096 114.3) (width 0.2) (layer F.Cu) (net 21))
 (segment (start 133.731 117.602) (end 133.096 116.967) (width 0.2) (layer F.Cu) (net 21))
 (segment (start 136.906 117.602) (end 133.731 117.602) (width 0.2) (layer F.Cu) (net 21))
 (segment (start 137.414 113.183) (end 137.414 117.094) (width 0.2) (layer F.Cu) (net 21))
 (segment (start 137.414 117.094) (end 136.906 117.602) (width 0.2) (layer F.Cu) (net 21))
 (segment (start 134.489811 111.883811) (end 133.818999 111.212999) (width 0.2) (layer F.Cu) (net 27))
 (segment (start 138.684 112.183) (end 138.384811 111.883811) (width 0.2) (layer F.Cu) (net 27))
 (segment (start 133.818999 111.212999) (end 132.969 110.363) (width 0.2) (layer F.Cu) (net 27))
 (segment (start 138.384811 111.883811) (end 134.489811 111.883811) (width 0.2) (layer F.Cu) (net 27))
 (segment (start 138.684 113.183) (end 138.684 112.183) (width 0.2) (layer F.Cu) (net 27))
 (segment (start 141.4867 114.383) (end 141.4867 113.308) (width 0.2) (layer B.Cu) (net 27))
 (segment (start 140.7007 112.522) (end 135.1534 112.522) (width 0.2) (layer B.Cu) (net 27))
 (segment (start 135.1534 112.522) (end 132.9944 110.363) (width 0.2) (layer B.Cu) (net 27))
 (segment (start 141.4867 113.308) (end 140.7007 112.522) (width 0.2) (layer B.Cu) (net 27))
 (segment (start 136.7028 111.5568) (end 135.509 110.363) (width 0.2) (layer F.Cu) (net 26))
 (segment (start 139.954 112.183) (end 139.3278 111.5568) (width 0.2) (layer F.Cu) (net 26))
 (segment (start 139.954 113.183) (end 139.954 112.183) (width 0.2) (layer F.Cu) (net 26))
 (segment (start 139.3278 111.5568) (end 136.7028 111.5568) (width 0.2) (layer F.Cu) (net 26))
 (segment (start 141.2494 112.014) (end 137.1854 112.014) (width 0.2) (layer B.Cu) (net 26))
 (segment (start 142.1367 112.9013) (end 141.2494 112.014) (width 0.2) (layer B.Cu) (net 26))
 (segment (start 142.1367 114.383) (end 142.1367 112.9013) (width 0.2) (layer B.Cu) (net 26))
 (segment (start 137.1854 112.014) (end 135.5344 110.363) (width 0.2) (layer B.Cu) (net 26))
 (segment (start 141.224 113.183) (end 141.224 112.772881) (width 0.2) (layer F.Cu) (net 25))
 (segment (start 141.224 112.772881) (end 139.550719 111.0996) (width 0.2) (layer F.Cu) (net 25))
 (segment (start 139.550719 111.0996) (end 138.7856 111.0996) (width 0.2) (layer F.Cu) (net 25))
 (segment (start 138.7856 111.0996) (end 138.049 110.363) (width 0.2) (layer F.Cu) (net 25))
 (segment (start 139.2174 111.506) (end 138.0744 110.363) (width 0.2) (layer B.Cu) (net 25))
 (segment (start 142.7867 114.383) (end 142.7867 112.6623) (width 0.2) (layer B.Cu) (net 25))
 (segment (start 142.7867 112.6623) (end 141.6304 111.506) (width 0.2) (layer B.Cu) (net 25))
 (segment (start 141.6304 111.506) (end 139.2174 111.506) (width 0.2) (layer B.Cu) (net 25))
 (segment (start 142.494 112.268) (end 141.438999 111.212999) (width 0.2) (layer F.Cu) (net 24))
 (segment (start 141.438999 111.212999) (end 140.589 110.363) (width 0.2) (layer F.Cu) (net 24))
 (segment (start 142.494 113.183) (end 142.494 112.268) (width 0.2) (layer F.Cu) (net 24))
 (segment (start 143.4367 114.383) (end 143.4367 112.4233) (width 0.2) (layer B.Cu) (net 24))
 (segment (start 143.4367 112.4233) (end 141.3764 110.363) (width 0.2) (layer B.Cu) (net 24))
 (segment (start 141.3764 110.363) (end 140.6144 110.363) (width 0.2) (layer B.Cu) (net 24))
 (segment (start 143.764 110.998) (end 143.129 110.363) (width 0.2) (layer F.Cu) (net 23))
 (segment (start 143.764 113.183) (end 143.764 110.998) (width 0.2) (layer F.Cu) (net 23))
 (segment (start 144.0867 111.2953) (end 143.1544 110.363) (width 0.2) (layer B.Cu) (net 23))
 (segment (start 144.0867 114.383) (end 144.0867 111.2953) (width 0.2) (layer B.Cu) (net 23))
 (segment (start 145.034 113.183) (end 145.034 110.998) (width 0.2) (layer F.Cu) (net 22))
 (segment (start 145.034 110.998) (end 145.669 110.363) (width 0.2) (layer F.Cu) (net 22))
 (segment (start 144.7367 111.3207) (end 145.6944 110.363) (width 0.2) (layer B.Cu) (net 22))
 (segment (start 144.7367 114.383) (end 144.7367 111.3207) (width 0.2) (layer B.Cu) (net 22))
 (segment (start 147.359001 111.212999) (end 148.209 110.363) (width 0.2) (layer F.Cu) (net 20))
 (segment (start 146.304 112.268) (end 147.359001 111.212999) (width 0.2) (layer F.Cu) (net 20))
 (segment (start 146.304 113.183) (end 146.304 112.268) (width 0.2) (layer F.Cu) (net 20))
 (segment (start 147.4724 110.363) (end 148.2344 110.363) (width 0.2) (layer B.Cu) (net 20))
 (segment (start 145.3867 112.4487) (end 147.4724 110.363) (width 0.2) (layer B.Cu) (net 20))
 (segment (start 145.3867 114.383) (end 145.3867 112.4487) (width 0.2) (layer B.Cu) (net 20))
 (segment (start 149.9616 110.363) (end 150.749 110.363) (width 0.2) (layer F.Cu) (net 17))
 (segment (start 147.574 113.183) (end 147.574 112.7506) (width 0.2) (layer F.Cu) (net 17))
 (segment (start 147.574 112.7506) (end 149.9616 110.363) (width 0.2) (layer F.Cu) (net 17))
 (segment (start 149.6314 111.506) (end 150.7744 110.363) (width 0.2) (layer B.Cu) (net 17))
 (segment (start 146.0367 112.6877) (end 147.2184 111.506) (width 0.2) (layer B.Cu) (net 17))
 (segment (start 146.0367 114.383) (end 146.0367 112.6877) (width 0.2) (layer B.Cu) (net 17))
 (segment (start 147.2184 111.506) (end 149.6314 111.506) (width 0.2) (layer B.Cu) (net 17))
 (segment (start 146.6867 112.9267) (end 147.5994 112.014) (width 0.2) (layer B.Cu) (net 16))
 (segment (start 146.6867 114.383) (end 146.6867 112.9267) (width 0.2) (layer B.Cu) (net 16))
 (segment (start 151.6634 112.014) (end 153.3144 110.363) (width 0.2) (layer B.Cu) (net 16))
 (segment (start 147.5994 112.014) (end 151.6634 112.014) (width 0.2) (layer B.Cu) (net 16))
 (segment (start 152.439001 111.212999) (end 153.289 110.363) (width 0.2) (layer F.Cu) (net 16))
 (segment (start 152.146 111.506) (end 152.439001 111.212999) (width 0.2) (layer F.Cu) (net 16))
 (segment (start 149.4536 111.506) (end 152.146 111.506) (width 0.2) (layer F.Cu) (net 16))
 (segment (start 148.844 113.183) (end 148.844 112.1156) (width 0.2) (layer F.Cu) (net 16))
 (segment (start 148.844 112.1156) (end 149.4536 111.506) (width 0.2) (layer F.Cu) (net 16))
 (segment (start 150.622 111.8616) (end 154.3304 111.8616) (width 0.2) (layer F.Cu) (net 15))
 (segment (start 150.114 113.183) (end 150.114 112.3696) (width 0.2) (layer F.Cu) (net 15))
 (segment (start 150.114 112.3696) (end 150.622 111.8616) (width 0.2) (layer F.Cu) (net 15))
 (segment (start 154.3304 111.8616) (end 154.979001 111.212999) (width 0.2) (layer F.Cu) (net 15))
 (segment (start 154.979001 111.212999) (end 155.829 110.363) (width 0.2) (layer F.Cu) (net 15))
 (segment (start 147.3367 114.383) (end 147.3367 113.1657) (width 0.2) (layer B.Cu) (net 15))
 (segment (start 147.9804 112.522) (end 153.6954 112.522) (width 0.2) (layer B.Cu) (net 15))
 (segment (start 153.6954 112.522) (end 155.8544 110.363) (width 0.2) (layer B.Cu) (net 15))
 (segment (start 147.3367 113.1657) (end 147.9804 112.522) (width 0.2) (layer B.Cu) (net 15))
 (via (at 155.702 114.3) (size 0.8) (drill 0.4) (layers F.Cu B.Cu) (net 19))
 (segment (start 147.9867 114.383) (end 147.9867 113.308) (width 0.2) (layer B.Cu) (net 19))
 (segment (start 147.9867 113.308) (end 148.2647 113.03) (width 0.2) (layer B.Cu) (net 19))
 (segment (start 148.2647 113.03) (end 155.7274 113.03) (width 0.2) (layer B.Cu) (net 19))
 (segment (start 155.7274 113.03) (end 158.3944 110.363) (width 0.2) (layer B.Cu) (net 19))
 (segment (start 155.702 113.0554) (end 155.7274 113.03) (width 0.2) (layer B.Cu) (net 19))
 (segment (start 155.702 114.3) (end 155.702 113.0554) (width 0.2) (layer B.Cu) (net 19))
 (segment (start 155.702 117.094) (end 155.702 114.3) (width 0.2) (layer F.Cu) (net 19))
 (segment (start 155.194 117.602) (end 155.702 117.094) (width 0.2) (layer F.Cu) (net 19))
 (segment (start 151.892 117.602) (end 155.194 117.602) (width 0.2) (layer F.Cu) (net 19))
 (segment (start 151.384 113.183) (end 151.384 117.094) (width 0.2) (layer F.Cu) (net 19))
 (segment (start 151.384 117.094) (end 151.892 117.602) (width 0.2) (layer F.Cu) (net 19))
 (segment (start 152.654 113.183) (end 158.089 113.183) (width 0.2) (layer F.Cu) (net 18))
 (segment (start 158.089 113.183) (end 160.909 110.363) (width 0.2) (layer F.Cu) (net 18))
 (segment (start 155.7274 115.57) (end 160.9344 110.363) (width 0.2) (layer B.Cu) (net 18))
 (segment (start 148.6367 114.383) (end 149.8237 115.57) (width 0.2) (layer B.Cu) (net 18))
 (segment (start 149.8237 115.57) (end 155.7274 115.57) (width 0.2) (layer B.Cu) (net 18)))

